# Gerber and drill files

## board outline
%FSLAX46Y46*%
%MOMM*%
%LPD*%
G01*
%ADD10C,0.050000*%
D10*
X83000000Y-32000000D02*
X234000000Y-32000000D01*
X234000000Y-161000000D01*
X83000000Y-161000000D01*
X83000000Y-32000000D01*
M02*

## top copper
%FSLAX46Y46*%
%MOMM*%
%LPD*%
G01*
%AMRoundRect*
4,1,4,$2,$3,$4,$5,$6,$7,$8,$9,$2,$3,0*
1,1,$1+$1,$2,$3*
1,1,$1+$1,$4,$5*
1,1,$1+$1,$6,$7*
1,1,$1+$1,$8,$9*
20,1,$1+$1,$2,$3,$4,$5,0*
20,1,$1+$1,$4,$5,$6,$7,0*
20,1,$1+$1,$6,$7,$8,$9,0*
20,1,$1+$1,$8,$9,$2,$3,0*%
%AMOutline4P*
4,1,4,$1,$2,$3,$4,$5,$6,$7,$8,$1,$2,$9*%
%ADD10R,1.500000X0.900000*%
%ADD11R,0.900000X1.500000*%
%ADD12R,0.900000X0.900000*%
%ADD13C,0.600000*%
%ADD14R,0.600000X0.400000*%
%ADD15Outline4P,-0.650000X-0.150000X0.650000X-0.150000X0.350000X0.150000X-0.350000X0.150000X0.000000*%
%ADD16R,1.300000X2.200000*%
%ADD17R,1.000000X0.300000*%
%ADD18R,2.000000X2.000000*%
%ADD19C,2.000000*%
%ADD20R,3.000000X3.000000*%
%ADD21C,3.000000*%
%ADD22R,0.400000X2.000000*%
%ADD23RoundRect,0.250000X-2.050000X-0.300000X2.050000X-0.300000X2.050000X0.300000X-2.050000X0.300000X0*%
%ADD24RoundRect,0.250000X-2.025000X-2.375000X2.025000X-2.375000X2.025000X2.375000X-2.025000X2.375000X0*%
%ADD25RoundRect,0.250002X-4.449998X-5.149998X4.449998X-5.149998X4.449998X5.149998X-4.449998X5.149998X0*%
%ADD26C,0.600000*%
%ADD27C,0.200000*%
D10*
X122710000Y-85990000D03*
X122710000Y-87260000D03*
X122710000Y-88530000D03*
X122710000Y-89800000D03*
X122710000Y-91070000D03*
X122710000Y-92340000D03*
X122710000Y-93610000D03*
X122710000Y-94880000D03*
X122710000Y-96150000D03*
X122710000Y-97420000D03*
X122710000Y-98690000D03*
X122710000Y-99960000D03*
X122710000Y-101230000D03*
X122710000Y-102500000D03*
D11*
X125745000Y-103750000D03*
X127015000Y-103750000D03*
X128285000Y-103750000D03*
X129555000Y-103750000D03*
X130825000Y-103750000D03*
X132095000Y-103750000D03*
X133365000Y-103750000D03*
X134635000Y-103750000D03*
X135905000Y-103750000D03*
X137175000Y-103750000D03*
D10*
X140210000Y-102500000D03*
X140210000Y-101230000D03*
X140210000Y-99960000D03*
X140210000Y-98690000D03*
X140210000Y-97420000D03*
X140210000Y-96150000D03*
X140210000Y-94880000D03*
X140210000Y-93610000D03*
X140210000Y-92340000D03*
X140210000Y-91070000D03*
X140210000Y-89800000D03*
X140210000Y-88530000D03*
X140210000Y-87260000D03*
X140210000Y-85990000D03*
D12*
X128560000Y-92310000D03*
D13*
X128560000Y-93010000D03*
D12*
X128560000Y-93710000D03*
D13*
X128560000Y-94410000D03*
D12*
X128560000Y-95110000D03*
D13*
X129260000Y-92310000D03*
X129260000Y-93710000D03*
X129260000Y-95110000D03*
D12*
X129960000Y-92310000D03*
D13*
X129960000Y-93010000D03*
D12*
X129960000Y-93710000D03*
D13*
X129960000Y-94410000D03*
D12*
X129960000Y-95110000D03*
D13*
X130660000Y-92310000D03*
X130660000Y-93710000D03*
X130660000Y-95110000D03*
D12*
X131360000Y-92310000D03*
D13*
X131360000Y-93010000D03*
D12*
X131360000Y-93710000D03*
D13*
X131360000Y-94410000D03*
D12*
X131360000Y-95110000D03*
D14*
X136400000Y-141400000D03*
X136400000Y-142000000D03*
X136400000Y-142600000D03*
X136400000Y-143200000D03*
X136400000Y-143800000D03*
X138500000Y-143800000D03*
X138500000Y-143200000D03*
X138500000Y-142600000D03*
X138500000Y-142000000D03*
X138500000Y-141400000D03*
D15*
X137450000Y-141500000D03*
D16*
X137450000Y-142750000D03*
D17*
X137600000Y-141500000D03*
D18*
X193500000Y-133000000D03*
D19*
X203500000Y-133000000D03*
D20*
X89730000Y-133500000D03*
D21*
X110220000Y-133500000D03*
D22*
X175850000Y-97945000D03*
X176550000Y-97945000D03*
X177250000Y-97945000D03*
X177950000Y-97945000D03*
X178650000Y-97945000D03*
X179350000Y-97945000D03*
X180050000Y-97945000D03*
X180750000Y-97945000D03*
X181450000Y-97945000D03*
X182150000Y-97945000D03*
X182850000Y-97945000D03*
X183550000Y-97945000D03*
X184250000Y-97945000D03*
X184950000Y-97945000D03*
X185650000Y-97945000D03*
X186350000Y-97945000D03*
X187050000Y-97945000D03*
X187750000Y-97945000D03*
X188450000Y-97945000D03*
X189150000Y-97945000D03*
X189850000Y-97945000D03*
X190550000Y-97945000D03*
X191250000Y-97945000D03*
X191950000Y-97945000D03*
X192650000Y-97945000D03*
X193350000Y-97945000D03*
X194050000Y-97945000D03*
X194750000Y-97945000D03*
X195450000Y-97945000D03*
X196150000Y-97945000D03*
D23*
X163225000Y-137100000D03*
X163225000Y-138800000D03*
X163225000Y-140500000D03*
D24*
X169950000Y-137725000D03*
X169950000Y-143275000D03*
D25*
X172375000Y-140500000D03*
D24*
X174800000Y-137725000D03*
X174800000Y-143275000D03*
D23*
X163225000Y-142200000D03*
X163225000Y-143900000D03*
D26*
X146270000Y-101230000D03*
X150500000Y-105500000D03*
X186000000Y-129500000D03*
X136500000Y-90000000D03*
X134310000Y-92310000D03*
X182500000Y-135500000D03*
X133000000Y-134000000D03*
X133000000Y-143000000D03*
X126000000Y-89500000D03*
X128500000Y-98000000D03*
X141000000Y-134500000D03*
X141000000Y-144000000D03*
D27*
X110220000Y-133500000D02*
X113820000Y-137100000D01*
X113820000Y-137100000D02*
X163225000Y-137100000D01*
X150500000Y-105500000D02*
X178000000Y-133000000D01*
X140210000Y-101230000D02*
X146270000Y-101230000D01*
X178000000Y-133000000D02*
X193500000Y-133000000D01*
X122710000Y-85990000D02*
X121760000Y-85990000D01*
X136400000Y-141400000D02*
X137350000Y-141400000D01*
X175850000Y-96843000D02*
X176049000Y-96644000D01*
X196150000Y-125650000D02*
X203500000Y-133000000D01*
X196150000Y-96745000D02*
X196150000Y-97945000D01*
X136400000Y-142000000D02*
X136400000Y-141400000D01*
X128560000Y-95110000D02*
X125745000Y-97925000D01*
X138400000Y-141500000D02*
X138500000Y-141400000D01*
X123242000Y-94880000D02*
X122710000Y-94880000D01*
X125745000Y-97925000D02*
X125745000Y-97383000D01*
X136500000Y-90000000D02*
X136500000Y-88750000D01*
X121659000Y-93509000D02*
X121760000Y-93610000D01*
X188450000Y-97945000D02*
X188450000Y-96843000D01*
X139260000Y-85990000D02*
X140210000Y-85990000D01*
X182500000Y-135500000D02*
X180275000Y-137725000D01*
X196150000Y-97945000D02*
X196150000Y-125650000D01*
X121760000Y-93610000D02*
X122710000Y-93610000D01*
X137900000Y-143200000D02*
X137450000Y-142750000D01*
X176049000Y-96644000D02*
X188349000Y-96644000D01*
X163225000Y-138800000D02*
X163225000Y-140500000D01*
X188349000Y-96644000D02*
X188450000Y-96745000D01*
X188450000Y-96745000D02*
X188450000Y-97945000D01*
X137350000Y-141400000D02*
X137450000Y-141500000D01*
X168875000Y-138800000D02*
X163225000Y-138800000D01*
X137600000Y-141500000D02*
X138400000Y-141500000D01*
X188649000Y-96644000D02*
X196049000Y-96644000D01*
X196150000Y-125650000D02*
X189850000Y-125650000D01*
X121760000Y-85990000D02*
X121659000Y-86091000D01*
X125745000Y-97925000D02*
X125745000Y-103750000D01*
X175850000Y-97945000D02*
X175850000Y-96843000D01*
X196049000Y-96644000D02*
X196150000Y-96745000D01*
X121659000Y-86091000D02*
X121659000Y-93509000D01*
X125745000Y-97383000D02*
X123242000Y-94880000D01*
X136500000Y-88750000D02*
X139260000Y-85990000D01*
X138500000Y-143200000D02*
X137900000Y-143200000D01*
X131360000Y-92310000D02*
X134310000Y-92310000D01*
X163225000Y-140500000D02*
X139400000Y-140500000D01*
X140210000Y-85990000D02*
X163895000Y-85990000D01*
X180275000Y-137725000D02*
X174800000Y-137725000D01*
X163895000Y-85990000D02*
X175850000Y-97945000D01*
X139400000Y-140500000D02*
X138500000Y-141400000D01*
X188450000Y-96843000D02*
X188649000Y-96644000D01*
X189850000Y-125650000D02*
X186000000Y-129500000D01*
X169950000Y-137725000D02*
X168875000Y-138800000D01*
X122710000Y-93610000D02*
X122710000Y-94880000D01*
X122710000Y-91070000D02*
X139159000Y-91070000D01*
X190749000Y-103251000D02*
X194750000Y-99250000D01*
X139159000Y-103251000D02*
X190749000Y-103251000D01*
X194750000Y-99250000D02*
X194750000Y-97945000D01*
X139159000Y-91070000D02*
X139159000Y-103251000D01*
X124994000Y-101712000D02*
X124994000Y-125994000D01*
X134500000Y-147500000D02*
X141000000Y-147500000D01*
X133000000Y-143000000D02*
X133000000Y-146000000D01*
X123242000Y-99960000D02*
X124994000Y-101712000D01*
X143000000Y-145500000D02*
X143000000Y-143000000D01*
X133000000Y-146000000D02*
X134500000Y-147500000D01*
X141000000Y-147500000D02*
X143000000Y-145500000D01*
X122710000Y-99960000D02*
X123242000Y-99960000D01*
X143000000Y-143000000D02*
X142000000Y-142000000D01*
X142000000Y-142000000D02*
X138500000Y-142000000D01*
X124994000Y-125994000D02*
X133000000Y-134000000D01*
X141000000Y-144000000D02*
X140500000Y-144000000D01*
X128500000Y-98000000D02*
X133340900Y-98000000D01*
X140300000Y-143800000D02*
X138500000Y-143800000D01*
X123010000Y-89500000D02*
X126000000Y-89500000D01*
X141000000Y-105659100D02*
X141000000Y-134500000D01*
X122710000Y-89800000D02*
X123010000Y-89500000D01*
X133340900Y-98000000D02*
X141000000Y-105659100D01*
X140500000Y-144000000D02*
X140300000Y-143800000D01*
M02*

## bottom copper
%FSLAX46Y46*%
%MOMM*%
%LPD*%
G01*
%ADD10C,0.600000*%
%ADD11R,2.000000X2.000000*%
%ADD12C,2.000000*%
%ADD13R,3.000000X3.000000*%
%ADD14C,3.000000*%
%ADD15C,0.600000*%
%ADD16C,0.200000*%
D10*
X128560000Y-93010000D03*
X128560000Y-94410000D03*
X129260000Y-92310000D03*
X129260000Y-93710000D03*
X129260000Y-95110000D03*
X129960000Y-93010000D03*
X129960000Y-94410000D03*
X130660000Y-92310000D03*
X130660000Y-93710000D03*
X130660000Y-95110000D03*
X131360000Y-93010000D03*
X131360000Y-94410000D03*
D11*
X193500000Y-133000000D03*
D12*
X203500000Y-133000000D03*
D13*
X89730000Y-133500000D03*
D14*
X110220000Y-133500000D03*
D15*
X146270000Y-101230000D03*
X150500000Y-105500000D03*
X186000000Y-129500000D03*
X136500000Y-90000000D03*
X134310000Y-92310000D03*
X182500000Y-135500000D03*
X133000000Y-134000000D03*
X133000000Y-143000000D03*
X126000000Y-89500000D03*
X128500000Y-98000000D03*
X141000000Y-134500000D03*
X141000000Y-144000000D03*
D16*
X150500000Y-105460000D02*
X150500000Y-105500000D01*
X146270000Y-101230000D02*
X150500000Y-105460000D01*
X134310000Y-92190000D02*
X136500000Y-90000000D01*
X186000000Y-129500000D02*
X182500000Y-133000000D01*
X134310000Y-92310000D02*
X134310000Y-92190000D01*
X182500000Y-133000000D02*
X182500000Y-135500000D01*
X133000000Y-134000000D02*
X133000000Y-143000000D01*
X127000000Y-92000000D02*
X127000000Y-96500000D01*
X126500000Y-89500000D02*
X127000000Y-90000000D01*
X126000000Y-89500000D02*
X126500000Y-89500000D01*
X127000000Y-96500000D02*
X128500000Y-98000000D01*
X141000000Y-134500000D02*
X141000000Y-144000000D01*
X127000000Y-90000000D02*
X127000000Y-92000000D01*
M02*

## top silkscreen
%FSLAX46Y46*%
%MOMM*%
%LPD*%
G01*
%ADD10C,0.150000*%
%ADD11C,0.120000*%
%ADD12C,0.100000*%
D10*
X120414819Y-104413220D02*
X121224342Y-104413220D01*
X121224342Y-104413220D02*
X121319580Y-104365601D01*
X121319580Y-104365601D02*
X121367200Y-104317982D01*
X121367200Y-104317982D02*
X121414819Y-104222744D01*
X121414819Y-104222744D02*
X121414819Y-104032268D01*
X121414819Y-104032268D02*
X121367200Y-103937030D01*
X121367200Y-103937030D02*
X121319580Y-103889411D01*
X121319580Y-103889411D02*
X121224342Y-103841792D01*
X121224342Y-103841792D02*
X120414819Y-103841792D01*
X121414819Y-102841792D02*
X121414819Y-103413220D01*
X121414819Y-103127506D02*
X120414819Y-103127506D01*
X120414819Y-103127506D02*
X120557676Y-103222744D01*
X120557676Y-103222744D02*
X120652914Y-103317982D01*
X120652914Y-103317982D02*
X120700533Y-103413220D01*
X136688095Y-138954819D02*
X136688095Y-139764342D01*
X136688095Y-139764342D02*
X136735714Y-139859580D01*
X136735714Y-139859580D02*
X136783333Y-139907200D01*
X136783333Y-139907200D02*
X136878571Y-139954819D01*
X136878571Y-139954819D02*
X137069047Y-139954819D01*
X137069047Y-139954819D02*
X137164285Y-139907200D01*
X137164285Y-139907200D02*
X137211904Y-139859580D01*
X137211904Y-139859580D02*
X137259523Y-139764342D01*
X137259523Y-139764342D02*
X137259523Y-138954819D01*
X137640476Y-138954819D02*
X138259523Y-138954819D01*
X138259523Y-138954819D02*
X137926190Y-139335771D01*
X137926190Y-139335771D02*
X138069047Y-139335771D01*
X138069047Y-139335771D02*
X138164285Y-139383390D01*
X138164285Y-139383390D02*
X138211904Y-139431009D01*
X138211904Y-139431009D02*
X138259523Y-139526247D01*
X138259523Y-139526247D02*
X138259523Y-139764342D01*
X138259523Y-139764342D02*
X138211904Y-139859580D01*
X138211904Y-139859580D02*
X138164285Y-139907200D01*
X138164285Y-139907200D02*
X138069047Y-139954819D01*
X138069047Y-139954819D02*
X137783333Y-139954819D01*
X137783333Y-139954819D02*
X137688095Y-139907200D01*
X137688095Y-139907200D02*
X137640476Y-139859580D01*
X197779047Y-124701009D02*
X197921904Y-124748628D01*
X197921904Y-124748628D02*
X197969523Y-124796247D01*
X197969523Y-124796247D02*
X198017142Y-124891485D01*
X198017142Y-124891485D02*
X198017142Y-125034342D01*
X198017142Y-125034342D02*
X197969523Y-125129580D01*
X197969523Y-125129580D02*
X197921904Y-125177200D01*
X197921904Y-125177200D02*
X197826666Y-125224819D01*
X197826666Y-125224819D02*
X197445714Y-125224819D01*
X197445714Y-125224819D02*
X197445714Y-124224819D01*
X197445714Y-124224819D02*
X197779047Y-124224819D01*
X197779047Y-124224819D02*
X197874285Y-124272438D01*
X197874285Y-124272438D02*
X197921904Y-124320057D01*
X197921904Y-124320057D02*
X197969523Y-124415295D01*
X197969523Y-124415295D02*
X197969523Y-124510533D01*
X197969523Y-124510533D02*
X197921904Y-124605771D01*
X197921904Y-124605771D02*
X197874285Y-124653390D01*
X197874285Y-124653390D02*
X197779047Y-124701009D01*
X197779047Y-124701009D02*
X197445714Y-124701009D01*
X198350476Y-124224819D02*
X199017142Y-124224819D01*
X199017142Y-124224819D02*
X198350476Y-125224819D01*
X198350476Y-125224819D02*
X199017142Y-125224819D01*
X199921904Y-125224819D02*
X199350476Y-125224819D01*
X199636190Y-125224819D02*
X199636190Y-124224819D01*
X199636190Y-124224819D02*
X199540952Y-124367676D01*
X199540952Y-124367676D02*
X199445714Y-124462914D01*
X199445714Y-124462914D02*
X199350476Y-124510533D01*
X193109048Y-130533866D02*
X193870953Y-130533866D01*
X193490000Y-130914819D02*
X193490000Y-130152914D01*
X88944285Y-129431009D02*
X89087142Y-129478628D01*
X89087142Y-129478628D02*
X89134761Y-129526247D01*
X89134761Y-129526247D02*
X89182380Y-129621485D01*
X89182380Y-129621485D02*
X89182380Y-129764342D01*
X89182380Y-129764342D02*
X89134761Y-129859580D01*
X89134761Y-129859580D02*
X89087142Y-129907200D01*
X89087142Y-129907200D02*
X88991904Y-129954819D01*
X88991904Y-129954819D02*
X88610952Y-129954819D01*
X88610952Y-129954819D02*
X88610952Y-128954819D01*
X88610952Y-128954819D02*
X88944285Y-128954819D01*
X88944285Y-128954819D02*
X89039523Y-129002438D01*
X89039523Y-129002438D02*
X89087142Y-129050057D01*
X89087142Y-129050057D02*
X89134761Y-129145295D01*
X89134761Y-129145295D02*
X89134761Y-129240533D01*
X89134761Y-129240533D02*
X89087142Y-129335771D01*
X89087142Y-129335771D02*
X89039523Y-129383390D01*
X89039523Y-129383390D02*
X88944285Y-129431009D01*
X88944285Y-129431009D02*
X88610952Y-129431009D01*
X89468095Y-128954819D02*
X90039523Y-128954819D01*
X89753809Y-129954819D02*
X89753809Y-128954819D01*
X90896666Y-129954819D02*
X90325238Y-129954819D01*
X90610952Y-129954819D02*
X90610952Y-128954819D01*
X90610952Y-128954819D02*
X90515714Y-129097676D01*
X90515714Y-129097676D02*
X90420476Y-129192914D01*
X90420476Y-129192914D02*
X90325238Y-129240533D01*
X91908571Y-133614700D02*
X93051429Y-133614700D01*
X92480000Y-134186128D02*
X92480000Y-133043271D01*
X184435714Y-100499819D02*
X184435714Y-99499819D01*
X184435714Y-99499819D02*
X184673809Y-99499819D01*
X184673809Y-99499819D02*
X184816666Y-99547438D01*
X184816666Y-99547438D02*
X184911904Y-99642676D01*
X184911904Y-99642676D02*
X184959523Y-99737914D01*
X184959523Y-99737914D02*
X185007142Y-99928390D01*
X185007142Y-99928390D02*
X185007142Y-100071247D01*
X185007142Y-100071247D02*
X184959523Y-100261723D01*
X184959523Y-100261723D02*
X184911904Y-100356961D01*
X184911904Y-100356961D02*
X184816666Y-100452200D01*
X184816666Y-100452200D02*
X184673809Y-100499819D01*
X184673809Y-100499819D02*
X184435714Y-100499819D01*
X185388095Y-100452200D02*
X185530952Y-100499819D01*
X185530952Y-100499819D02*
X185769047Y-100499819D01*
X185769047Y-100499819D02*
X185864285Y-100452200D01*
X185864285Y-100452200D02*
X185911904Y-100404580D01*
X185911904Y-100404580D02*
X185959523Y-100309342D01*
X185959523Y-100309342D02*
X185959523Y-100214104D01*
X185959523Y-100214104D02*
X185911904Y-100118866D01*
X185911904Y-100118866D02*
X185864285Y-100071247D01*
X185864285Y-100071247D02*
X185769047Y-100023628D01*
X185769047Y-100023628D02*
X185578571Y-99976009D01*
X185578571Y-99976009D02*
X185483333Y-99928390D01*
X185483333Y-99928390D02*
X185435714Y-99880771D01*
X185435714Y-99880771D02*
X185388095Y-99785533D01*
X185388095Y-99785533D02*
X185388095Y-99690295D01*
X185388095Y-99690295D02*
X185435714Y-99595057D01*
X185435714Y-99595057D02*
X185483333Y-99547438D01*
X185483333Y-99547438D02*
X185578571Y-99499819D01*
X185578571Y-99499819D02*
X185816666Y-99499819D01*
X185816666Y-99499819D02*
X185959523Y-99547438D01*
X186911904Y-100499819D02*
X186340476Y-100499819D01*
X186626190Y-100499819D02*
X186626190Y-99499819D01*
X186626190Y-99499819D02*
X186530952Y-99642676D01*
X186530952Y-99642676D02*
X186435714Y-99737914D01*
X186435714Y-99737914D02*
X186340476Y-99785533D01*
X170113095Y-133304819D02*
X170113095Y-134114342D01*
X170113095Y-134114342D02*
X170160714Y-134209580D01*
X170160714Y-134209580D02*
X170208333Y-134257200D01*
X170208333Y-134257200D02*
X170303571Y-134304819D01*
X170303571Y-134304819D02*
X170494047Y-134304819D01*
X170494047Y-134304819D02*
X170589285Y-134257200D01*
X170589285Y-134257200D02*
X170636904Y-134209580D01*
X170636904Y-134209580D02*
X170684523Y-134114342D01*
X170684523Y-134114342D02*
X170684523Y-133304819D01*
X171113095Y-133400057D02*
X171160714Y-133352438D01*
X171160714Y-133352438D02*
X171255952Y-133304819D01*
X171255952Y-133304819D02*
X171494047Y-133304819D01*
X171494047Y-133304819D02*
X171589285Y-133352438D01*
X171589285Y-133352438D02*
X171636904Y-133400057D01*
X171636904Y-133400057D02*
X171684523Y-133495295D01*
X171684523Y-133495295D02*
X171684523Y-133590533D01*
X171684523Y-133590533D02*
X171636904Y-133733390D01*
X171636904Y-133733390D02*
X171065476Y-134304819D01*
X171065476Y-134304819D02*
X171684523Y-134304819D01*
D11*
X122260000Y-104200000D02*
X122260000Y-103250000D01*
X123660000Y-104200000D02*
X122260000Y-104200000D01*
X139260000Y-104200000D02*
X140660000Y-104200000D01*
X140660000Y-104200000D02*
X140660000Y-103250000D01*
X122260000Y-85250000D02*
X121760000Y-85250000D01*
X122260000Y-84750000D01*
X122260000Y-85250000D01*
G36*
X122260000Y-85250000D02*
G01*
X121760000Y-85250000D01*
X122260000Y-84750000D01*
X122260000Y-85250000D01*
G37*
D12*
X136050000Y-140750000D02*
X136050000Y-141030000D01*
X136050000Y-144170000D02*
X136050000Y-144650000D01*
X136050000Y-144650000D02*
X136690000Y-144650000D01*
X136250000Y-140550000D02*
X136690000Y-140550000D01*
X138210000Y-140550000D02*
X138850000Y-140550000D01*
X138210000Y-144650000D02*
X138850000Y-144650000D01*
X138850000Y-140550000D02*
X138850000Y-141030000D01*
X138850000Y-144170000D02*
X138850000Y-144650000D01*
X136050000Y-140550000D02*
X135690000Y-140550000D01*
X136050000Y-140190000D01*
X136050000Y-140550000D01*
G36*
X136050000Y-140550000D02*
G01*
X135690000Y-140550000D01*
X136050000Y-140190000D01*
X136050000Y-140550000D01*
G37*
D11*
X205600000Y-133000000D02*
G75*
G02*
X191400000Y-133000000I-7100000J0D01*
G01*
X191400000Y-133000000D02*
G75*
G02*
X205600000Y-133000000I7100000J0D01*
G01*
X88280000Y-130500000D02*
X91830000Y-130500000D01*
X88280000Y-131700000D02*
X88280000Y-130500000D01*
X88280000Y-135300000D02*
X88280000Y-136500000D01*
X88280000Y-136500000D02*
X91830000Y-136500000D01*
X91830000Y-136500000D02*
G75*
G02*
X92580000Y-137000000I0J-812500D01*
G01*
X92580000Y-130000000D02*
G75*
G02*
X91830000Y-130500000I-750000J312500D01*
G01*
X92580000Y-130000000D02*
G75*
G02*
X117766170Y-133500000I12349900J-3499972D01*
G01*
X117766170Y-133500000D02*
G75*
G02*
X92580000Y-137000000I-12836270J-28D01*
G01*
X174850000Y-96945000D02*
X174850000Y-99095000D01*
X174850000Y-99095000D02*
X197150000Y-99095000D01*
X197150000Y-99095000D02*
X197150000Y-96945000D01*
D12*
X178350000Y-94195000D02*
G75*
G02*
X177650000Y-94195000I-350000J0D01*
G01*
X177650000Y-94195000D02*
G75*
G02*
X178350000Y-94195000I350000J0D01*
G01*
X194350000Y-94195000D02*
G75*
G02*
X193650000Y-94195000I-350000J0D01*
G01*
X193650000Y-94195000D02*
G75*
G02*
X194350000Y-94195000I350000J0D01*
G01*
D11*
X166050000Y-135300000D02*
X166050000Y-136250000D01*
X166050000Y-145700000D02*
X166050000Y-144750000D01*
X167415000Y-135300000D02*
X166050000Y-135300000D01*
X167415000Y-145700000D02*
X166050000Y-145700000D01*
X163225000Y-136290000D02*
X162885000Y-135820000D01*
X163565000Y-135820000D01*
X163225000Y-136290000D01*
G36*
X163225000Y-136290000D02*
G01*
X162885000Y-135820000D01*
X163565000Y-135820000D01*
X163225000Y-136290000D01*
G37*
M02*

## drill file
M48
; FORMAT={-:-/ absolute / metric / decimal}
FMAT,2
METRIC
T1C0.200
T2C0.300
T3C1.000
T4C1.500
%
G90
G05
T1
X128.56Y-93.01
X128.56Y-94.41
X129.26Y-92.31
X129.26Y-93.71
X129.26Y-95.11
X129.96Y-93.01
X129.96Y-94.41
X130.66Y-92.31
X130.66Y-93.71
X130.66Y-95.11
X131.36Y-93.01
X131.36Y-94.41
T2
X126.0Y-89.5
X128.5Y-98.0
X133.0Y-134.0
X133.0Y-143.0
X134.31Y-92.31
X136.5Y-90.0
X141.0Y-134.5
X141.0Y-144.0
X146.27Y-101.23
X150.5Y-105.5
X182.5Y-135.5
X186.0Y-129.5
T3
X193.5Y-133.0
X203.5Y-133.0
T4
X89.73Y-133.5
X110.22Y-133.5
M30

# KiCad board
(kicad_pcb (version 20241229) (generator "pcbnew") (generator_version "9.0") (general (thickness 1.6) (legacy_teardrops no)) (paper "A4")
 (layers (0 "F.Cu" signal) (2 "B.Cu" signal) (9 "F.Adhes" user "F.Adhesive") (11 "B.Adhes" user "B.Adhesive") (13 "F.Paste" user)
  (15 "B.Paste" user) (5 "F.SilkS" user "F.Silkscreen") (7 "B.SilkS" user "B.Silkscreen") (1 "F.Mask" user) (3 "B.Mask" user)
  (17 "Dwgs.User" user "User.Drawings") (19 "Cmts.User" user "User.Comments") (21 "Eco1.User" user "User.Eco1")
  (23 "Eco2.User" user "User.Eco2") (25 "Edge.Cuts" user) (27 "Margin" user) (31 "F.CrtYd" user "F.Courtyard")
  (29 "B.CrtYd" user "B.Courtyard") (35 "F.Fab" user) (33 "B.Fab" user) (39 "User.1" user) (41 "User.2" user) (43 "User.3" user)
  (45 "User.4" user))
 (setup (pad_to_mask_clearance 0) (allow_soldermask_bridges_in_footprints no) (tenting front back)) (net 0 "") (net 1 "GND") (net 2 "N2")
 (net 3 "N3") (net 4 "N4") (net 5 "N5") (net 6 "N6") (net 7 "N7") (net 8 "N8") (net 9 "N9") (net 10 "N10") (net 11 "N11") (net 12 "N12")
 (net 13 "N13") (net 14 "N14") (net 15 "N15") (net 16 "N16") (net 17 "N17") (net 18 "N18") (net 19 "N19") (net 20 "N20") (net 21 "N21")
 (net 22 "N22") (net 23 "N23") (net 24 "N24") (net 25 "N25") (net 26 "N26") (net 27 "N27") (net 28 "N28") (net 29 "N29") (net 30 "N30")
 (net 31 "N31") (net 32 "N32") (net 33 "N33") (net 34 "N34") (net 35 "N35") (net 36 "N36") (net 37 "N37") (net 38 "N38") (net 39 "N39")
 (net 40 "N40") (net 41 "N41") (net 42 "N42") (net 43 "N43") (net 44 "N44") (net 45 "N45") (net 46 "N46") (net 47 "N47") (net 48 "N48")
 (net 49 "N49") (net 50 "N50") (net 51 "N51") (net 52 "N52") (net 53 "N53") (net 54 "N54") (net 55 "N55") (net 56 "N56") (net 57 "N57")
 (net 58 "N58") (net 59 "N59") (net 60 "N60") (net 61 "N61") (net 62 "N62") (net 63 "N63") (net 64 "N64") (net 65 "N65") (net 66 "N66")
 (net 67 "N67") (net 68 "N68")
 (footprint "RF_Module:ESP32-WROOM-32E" (layer "F.Cu") (at 131.46 91.25)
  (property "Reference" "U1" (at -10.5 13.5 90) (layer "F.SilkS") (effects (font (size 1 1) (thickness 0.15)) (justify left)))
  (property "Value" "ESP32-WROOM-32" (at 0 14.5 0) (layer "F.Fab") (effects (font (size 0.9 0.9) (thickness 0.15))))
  (fp_line (start -9.2 12.95) (end -9.2 12) (stroke (width 0.12) (type solid)) (layer "F.SilkS"))
  (fp_line (start -7.8 12.95) (end -9.2 12.95) (stroke (width 0.12) (type solid)) (layer "F.SilkS"))
  (fp_line (start 7.8 12.95) (end 9.2 12.95) (stroke (width 0.12) (type solid)) (layer "F.SilkS"))
  (fp_line (start 9.2 12.95) (end 9.2 12) (stroke (width 0.12) (type solid)) (layer "F.SilkS"))
  (fp_poly (pts (xy -9.2 -6) (xy -9.7 -6) (xy -9.2 -6.5) (xy -9.2 -6)) (stroke (width 0.12) (type solid)) (fill yes) (layer "F.SilkS"))
  (pad "1" smd rect (at -8.75 -5.26) (size 1.5 0.9) (layers "F.Cu" "F.Mask" "F.Paste") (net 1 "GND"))
  (pad "2" smd rect (at -8.75 -3.99) (size 1.5 0.9) (layers "F.Cu" "F.Mask" "F.Paste") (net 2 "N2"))
  (pad "3" smd rect (at -8.75 -2.72) (size 1.5 0.9) (layers "F.Cu" "F.Mask" "F.Paste") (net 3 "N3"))
  (pad "4" smd rect (at -8.75 -1.45) (size 1.5 0.9) (layers "F.Cu" "F.Mask" "F.Paste") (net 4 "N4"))
  (pad "5" smd rect (at -8.75 -0.18) (size 1.5 0.9) (layers "F.Cu" "F.Mask" "F.Paste") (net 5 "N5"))
  (pad "6" smd rect (at -8.75 1.09) (size 1.5 0.9) (layers "F.Cu" "F.Mask" "F.Paste") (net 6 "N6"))
  (pad "7" smd rect (at -8.75 2.36) (size 1.5 0.9) (layers "F.Cu" "F.Mask" "F.Paste") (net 1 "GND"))
  (pad "8" smd rect (at -8.75 3.63) (size 1.5 0.9) (layers "F.Cu" "F.Mask" "F.Paste") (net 1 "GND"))
  (pad "9" smd rect (at -8.75 4.9) (size 1.5 0.9) (layers "F.Cu" "F.Mask" "F.Paste") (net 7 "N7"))
  (pad "10" smd rect (at -8.75 6.17) (size 1.5 0.9) (layers "F.Cu" "F.Mask" "F.Paste") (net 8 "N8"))
  (pad "11" smd rect (at -8.75 7.44) (size 1.5 0.9) (layers "F.Cu" "F.Mask" "F.Paste") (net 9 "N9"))
  (pad "12" smd rect (at -8.75 8.71) (size 1.5 0.9) (layers "F.Cu" "F.Mask" "F.Paste") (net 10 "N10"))
  (pad "13" smd rect (at -8.75 9.98) (size 1.5 0.9) (layers "F.Cu" "F.Mask" "F.Paste") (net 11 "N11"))
  (pad "14" smd rect (at -8.75 11.25) (size 1.5 0.9) (layers "F.Cu" "F.Mask" "F.Paste") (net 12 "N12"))
  (pad "15" smd rect (at -5.715 12.5 90) (size 1.5 0.9) (layers "F.Cu" "F.Mask" "F.Paste") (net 1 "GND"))
  (pad "16" smd rect (at -4.445 12.5 90) (size 1.5 0.9) (layers "F.Cu" "F.Mask" "F.Paste") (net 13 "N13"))
  (pad "17" smd rect (at -3.175 12.5 90) (size 1.5 0.9) (layers "F.Cu" "F.Mask" "F.Paste") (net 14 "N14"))
  (pad "18" smd rect (at -1.905 12.5 90) (size 1.5 0.9) (layers "F.Cu" "F.Mask" "F.Paste") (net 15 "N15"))
  (pad "19" smd rect (at -0.635 12.5 90) (size 1.5 0.9) (layers "F.Cu" "F.Mask" "F.Paste") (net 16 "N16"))
  (pad "20" smd rect (at 0.635 12.5 90) (size 1.5 0.9) (layers "F.Cu" "F.Mask" "F.Paste") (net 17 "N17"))
  (pad "21" smd rect (at 1.905 12.5 90) (size 1.5 0.9) (layers "F.Cu" "F.Mask" "F.Paste") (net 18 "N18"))
  (pad "22" smd rect (at 3.175 12.5 90) (size 1.5 0.9) (layers "F.Cu" "F.Mask" "F.Paste") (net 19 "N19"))
  (pad "23" smd rect (at 4.445 12.5 90) (size 1.5 0.9) (layers "F.Cu" "F.Mask" "F.Paste") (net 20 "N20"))
  (pad "24" smd rect (at 5.715 12.5 90) (size 1.5 0.9) (layers "F.Cu" "F.Mask" "F.Paste") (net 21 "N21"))
  (pad "25" smd rect (at 8.75 11.25) (size 1.5 0.9) (layers "F.Cu" "F.Mask" "F.Paste") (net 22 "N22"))
  (pad "26" smd rect (at 8.75 9.98) (size 1.5 0.9) (layers "F.Cu" "F.Mask" "F.Paste") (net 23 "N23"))
  (pad "27" smd rect (at 8.75 8.71) (size 1.5 0.9) (layers "F.Cu" "F.Mask" "F.Paste") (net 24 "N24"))
  (pad "28" smd rect (at 8.75 7.44) (size 1.5 0.9) (layers "F.Cu" "F.Mask" "F.Paste") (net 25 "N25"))
  (pad "29" smd rect (at 8.75 6.17) (size 1.5 0.9) (layers "F.Cu" "F.Mask" "F.Paste") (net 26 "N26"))
  (pad "30" smd rect (at 8.75 4.9) (size 1.5 0.9) (layers "F.Cu" "F.Mask" "F.Paste") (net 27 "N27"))
  (pad "31" smd rect (at 8.75 3.63) (size 1.5 0.9) (layers "F.Cu" "F.Mask" "F.Paste") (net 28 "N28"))
  (pad "32" smd rect (at 8.75 2.36) (size 1.5 0.9) (layers "F.Cu" "F.Mask" "F.Paste") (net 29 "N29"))
  (pad "33" smd rect (at 8.75 1.09) (size 1.5 0.9) (layers "F.Cu" "F.Mask" "F.Paste") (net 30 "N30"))
  (pad "34" smd rect (at 8.75 -0.18) (size 1.5 0.9) (layers "F.Cu" "F.Mask" "F.Paste") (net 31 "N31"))
  (pad "35" smd rect (at 8.75 -1.45) (size 1.5 0.9) (layers "F.Cu" "F.Mask" "F.Paste") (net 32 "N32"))
  (pad "36" smd rect (at 8.75 -2.72) (size 1.5 0.9) (layers "F.Cu" "F.Mask" "F.Paste") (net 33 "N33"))
  (pad "37" smd rect (at 8.75 -3.99) (size 1.5 0.9) (layers "F.Cu" "F.Mask" "F.Paste") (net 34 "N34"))
  (pad "38" smd rect (at 8.75 -5.26) (size 1.5 0.9) (layers "F.Cu" "F.Mask" "F.Paste") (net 1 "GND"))
  (pad "39" smd rect (at -2.9 1.06) (size 0.9 0.9) (layers "F.Cu" "F.Mask" "F.Paste") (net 1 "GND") (zone_connect 2))
  (pad "39" thru_hole circle (at -2.9 1.76) (size 0.6 0.6) (drill 0.2) (layers "*.Cu" "*.Mask") (remove_unused_layers no) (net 1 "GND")
   (zone_connect 2))
  (pad "39" smd rect (at -2.9 2.46) (size 0.9 0.9) (layers "F.Cu" "F.Mask" "F.Paste") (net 1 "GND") (zone_connect 2))
  (pad "39" thru_hole circle (at -2.9 3.16) (size 0.6 0.6) (drill 0.2) (layers "*.Cu" "*.Mask") (remove_unused_layers no) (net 1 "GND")
   (zone_connect 2))
  (pad "39" smd rect (at -2.9 3.86) (size 0.9 0.9) (layers "F.Cu" "F.Mask" "F.Paste") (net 1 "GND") (zone_connect 2))
  (pad "39" thru_hole circle (at -2.2 1.06) (size 0.6 0.6) (drill 0.2) (layers "*.Cu" "*.Mask") (remove_unused_layers no) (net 1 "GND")
   (zone_connect 2))
  (pad "39" thru_hole circle (at -2.2 2.46) (size 0.6 0.6) (drill 0.2) (layers "*.Cu" "*.Mask") (remove_unused_layers no) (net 1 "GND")
   (zone_connect 2))
  (pad "39" thru_hole circle (at -2.2 3.86) (size 0.6 0.6) (drill 0.2) (layers "*.Cu" "*.Mask") (remove_unused_layers no) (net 1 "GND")
   (zone_connect 2))
  (pad "39" smd rect (at -1.5 1.06) (size 0.9 0.9) (layers "F.Cu" "F.Mask" "F.Paste") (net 1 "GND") (zone_connect 2))
  (pad "39" thru_hole circle (at -1.5 1.76) (size 0.6 0.6) (drill 0.2) (layers "*.Cu" "*.Mask") (remove_unused_layers no) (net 1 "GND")
   (zone_connect 2))
  (pad "39" smd rect (at -1.5 2.46) (size 0.9 0.9) (layers "F.Cu" "F.Mask" "F.Paste") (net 1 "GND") (zone_connect 2))
  (pad "39" thru_hole circle (at -1.5 3.16) (size 0.6 0.6) (drill 0.2) (layers "*.Cu" "*.Mask") (remove_unused_layers no) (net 1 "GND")
   (zone_connect 2))
  (pad "39" smd rect (at -1.5 3.86) (size 0.9 0.9) (layers "F.Cu" "F.Mask" "F.Paste") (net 1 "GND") (zone_connect 2))
  (pad "39" thru_hole circle (at -0.8 1.06) (size 0.6 0.6) (drill 0.2) (layers "*.Cu" "*.Mask") (remove_unused_layers no) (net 1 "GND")
   (zone_connect 2))
  (pad "39" thru_hole circle (at -0.8 2.46) (size 0.6 0.6) (drill 0.2) (layers "*.Cu" "*.Mask") (remove_unused_layers no) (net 1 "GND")
   (zone_connect 2))
  (pad "39" thru_hole circle (at -0.8 3.86) (size 0.6 0.6) (drill 0.2) (layers "*.Cu" "*.Mask") (remove_unused_layers no) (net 1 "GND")
   (zone_connect 2))
  (pad "39" smd rect (at -0.1 1.06) (size 0.9 0.9) (layers "F.Cu" "F.Mask" "F.Paste") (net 1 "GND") (zone_connect 2))
  (pad "39" thru_hole circle (at -0.1 1.76) (size 0.6 0.6) (drill 0.2) (layers "*.Cu" "*.Mask") (remove_unused_layers no) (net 1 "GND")
   (zone_connect 2))
  (pad "39" smd rect (at -0.1 2.46) (size 0.9 0.9) (layers "F.Cu" "F.Mask" "F.Paste") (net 1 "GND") (zone_connect 2))
  (pad "39" thru_hole circle (at -0.1 3.16) (size 0.6 0.6) (drill 0.2) (layers "*.Cu" "*.Mask") (remove_unused_layers no) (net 1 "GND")
   (zone_connect 2))
  (pad "39" smd rect (at -0.1 3.86) (size 0.9 0.9) (layers "F.Cu" "F.Mask" "F.Paste") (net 1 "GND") (zone_connect 2))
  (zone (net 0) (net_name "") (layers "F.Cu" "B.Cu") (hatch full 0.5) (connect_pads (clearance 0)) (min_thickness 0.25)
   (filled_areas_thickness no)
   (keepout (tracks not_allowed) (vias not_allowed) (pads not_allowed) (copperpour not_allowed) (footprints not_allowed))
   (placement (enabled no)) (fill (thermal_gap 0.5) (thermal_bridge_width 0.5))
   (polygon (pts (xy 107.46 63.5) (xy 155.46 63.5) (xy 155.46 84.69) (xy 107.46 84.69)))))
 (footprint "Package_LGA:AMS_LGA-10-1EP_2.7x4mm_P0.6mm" (layer "F.Cu") (at 137.45 142.6)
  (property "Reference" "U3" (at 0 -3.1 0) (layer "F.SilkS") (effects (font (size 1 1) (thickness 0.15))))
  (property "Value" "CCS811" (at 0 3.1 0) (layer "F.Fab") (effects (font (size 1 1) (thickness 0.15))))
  (fp_line (start -1.4 -1.85) (end -1.4 -1.57) (stroke (width 0.1) (type solid)) (layer "F.SilkS"))
  (fp_line (start -1.4 1.57) (end -1.4 2.05) (stroke (width 0.1) (type solid)) (layer "F.SilkS"))
  (fp_line (start -1.4 2.05) (end -0.76 2.05) (stroke (width 0.1) (type solid)) (layer "F.SilkS"))
  (fp_line (start -1.2 -2.05) (end -0.76 -2.05) (stroke (width 0.1) (type solid)) (layer "F.SilkS"))
  (fp_line (start 0.76 -2.05) (end 1.4 -2.05) (stroke (width 0.1) (type solid)) (layer "F.SilkS"))
  (fp_line (start 0.76 2.05) (end 1.4 2.05) (stroke (width 0.1) (type solid)) (layer "F.SilkS"))
  (fp_line (start 1.4 -2.05) (end 1.4 -1.57) (stroke (width 0.1) (type solid)) (layer "F.SilkS"))
  (fp_line (start 1.4 1.57) (end 1.4 2.05) (stroke (width 0.1) (type solid)) (layer "F.SilkS"))
  (fp_poly
   (pts (xy -1.4 -2.05) (xy -1.76 -2.05) (xy -1.4 -2.41) (xy -1.4 -2.05)) (stroke (width 0.1) (type solid)) (fill yes) (layer "F.SilkS"))
  (pad "1" smd rect (at -1.05 -1.2) (size 0.6 0.4) (layers "F.Cu" "F.Mask" "F.Paste") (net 1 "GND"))
  (pad "2" smd rect (at -1.05 -0.6) (size 0.6 0.4) (layers "F.Cu" "F.Mask" "F.Paste") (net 1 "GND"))
  (pad "3" smd rect (at -1.05 0) (size 0.6 0.4) (layers "F.Cu" "F.Mask" "F.Paste") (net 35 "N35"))
  (pad "4" smd rect (at -1.05 0.6) (size 0.6 0.4) (layers "F.Cu" "F.Mask" "F.Paste") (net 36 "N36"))
  (pad "5" smd rect (at -1.05 1.2) (size 0.6 0.4) (layers "F.Cu" "F.Mask" "F.Paste") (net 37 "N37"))
  (pad "6" smd rect (at 1.05 1.2) (size 0.6 0.4) (layers "F.Cu" "F.Mask" "F.Paste") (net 4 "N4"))
  (pad "7" smd rect (at 1.05 0.6) (size 0.6 0.4) (layers "F.Cu" "F.Mask" "F.Paste") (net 1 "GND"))
  (pad "8" smd rect (at 1.05 0) (size 0.6 0.4) (layers "F.Cu" "F.Mask" "F.Paste") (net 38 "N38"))
  (pad "9" smd rect (at 1.05 -0.6) (size 0.6 0.4) (layers "F.Cu" "F.Mask" "F.Paste") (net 10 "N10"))
  (pad "10" smd rect (at 1.05 -1.2) (size 0.6 0.4) (layers "F.Cu" "F.Mask" "F.Paste") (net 1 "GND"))
  (pad "11" smd trapezoid (at 0 -1.1) (size 1 0.3) (rect_delta 0 0.3) (layers "F.Cu" "F.Mask" "F.Paste") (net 1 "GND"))
  (pad "11" smd rect (at 0 0.15) (size 1.3 2.2) (layers "F.Cu" "F.Mask" "F.Paste") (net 1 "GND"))
  (pad "11" smd rect (at 0.15 -1.1) (size 1 0.3) (layers "F.Cu" "F.Mask" "F.Paste") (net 1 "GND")))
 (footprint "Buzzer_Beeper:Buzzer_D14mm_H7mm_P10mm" (layer "F.Cu") (at 193.5 133)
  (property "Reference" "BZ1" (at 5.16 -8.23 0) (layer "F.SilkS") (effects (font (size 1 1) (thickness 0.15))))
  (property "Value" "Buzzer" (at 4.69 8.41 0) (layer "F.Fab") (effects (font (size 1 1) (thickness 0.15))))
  (fp_circle (center 5 0) (end 12.1 0) (stroke (width 0.12) (type solid)) (fill no) (layer "F.SilkS"))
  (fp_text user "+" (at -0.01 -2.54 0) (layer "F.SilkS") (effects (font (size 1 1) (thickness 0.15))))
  (pad "1" thru_hole rect (at 0 0) (size 2 2) (drill 1) (layers "*.Cu" "*.Mask") (remove_unused_layers no) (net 23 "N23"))
  (pad "2" thru_hole circle (at 10 0) (size 2 2) (drill 1) (layers "*.Cu" "*.Mask") (remove_unused_layers no) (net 1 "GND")))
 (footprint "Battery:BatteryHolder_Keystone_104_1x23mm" (layer "F.Cu") (at 89.73 133.5)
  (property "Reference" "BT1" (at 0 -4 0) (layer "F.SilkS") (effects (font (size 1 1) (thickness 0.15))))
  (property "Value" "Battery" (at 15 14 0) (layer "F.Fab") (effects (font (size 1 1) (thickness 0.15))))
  (fp_line (start -1.45 -3) (end 2.1 -3) (stroke (width 0.12) (type solid)) (layer "F.SilkS"))
  (fp_line (start -1.45 -1.8) (end -1.45 -3) (stroke (width 0.12) (type solid)) (layer "F.SilkS"))
  (fp_line (start -1.45 1.8) (end -1.45 3) (stroke (width 0.12) (type solid)) (layer "F.SilkS"))
  (fp_line (start -1.45 3) (end 2.1 3) (stroke (width 0.12) (type solid)) (layer "F.SilkS"))
  (fp_arc (start 2.1 3) (mid 2.550694 3.136459) (end 2.85 3.5) (stroke (width 0.12) (type solid)) (layer "F.SilkS"))
  (fp_arc (start 2.85 -3.5) (mid 2.550694 -3.136459) (end 2.1 -3) (stroke (width 0.12) (type solid)) (layer "F.SilkS"))
  (fp_arc (start 2.85 -3.5) (mid 16.966716 -12.714122) (end 28.03617 0) (stroke (width 0.12) (type solid)) (layer "F.SilkS"))
  (fp_arc (start 28.03617 0) (mid 16.966716 12.714122) (end 2.85 3.5) (stroke (width 0.12) (type solid)) (layer "F.SilkS"))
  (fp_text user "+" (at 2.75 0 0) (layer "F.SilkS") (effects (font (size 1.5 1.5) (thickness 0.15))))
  (pad "1" thru_hole rect (at 0 0) (size 3 3) (drill 1.5) (layers "*.Cu" "*.Mask") (remove_unused_layers no) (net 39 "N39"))
  (pad "2" thru_hole circle (at 20.49 0) (size 3 3) (drill 1.5) (layers "*.Cu" "*.Mask") (remove_unused_layers no) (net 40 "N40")))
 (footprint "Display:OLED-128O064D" (layer "F.Cu") (at 186 97.945)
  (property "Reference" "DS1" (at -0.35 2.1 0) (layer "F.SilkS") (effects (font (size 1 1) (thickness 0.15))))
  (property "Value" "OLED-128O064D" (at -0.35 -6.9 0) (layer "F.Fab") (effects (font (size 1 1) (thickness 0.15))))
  (fp_line (start -11.15 -1) (end -11.15 1.15) (stroke (width 0.12) (type solid)) (layer "F.SilkS"))
  (fp_line (start -11.15 1.15) (end 11.15 1.15) (stroke (width 0.12) (type solid)) (layer "F.SilkS"))
  (fp_line (start 11.15 1.15) (end 11.15 -1) (stroke (width 0.12) (type solid)) (layer "F.SilkS"))
  (fp_circle (center -8 -3.75) (end -7.65 -3.75) (stroke (width 0.1) (type solid)) (fill no) (layer "F.SilkS"))
  (fp_circle (center 8 -3.75) (end 8.35 -3.75) (stroke (width 0.1) (type solid)) (fill no) (layer "F.SilkS"))
  (pad "1" smd rect (at -10.15 0) (size 0.4 2) (layers "F.Cu" "F.Mask" "F.Paste") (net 1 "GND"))
  (pad "2" smd rect (at -9.45 0) (size 0.4 2) (layers "F.Cu" "F.Mask" "F.Paste") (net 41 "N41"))
  (pad "3" smd rect (at -8.75 0) (size 0.4 2) (layers "F.Cu" "F.Mask" "F.Paste") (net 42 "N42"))
  (pad "4" smd rect (at -8.05 0) (size 0.4 2) (layers "F.Cu" "F.Mask" "F.Paste") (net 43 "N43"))
  (pad "5" smd rect (at -7.35 0) (size 0.4 2) (layers "F.Cu" "F.Mask" "F.Paste") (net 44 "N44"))
  (pad "6" smd rect (at -6.65 0) (size 0.4 2) (layers "F.Cu" "F.Mask" "F.Paste") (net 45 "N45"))
  (pad "7" smd rect (at -5.95 0) (size 0.4 2) (layers "F.Cu" "F.Mask" "F.Paste") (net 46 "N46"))
  (pad "8" smd rect (at -5.25 0) (size 0.4 2) (layers "F.Cu" "F.Mask" "F.Paste") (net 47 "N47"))
  (pad "9" smd rect (at -4.55 0) (size 0.4 2) (layers "F.Cu" "F.Mask" "F.Paste") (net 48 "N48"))
  (pad "10" smd rect (at -3.85 0) (size 0.4 2) (layers "F.Cu" "F.Mask" "F.Paste") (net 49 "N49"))
  (pad "11" smd rect (at -3.15 0) (size 0.4 2) (layers "F.Cu" "F.Mask" "F.Paste") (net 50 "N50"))
  (pad "12" smd rect (at -2.45 0) (size 0.4 2) (layers "F.Cu" "F.Mask" "F.Paste") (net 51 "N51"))
  (pad "13" smd rect (at -1.75 0) (size 0.4 2) (layers "F.Cu" "F.Mask" "F.Paste") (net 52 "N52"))
  (pad "14" smd rect (at -1.05 0) (size 0.4 2) (layers "F.Cu" "F.Mask" "F.Paste") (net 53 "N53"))
  (pad "15" smd rect (at -0.35 0) (size 0.4 2) (layers "F.Cu" "F.Mask" "F.Paste") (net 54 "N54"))
  (pad "16" smd rect (at 0.35 0) (size 0.4 2) (layers "F.Cu" "F.Mask" "F.Paste") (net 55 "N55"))
  (pad "17" smd rect (at 1.05 0) (size 0.4 2) (layers "F.Cu" "F.Mask" "F.Paste") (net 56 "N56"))
  (pad "18" smd rect (at 1.75 0) (size 0.4 2) (layers "F.Cu" "F.Mask" "F.Paste") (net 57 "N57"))
  (pad "19" smd rect (at 2.45 0) (size 0.4 2) (layers "F.Cu" "F.Mask" "F.Paste") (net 1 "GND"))
  (pad "20" smd rect (at 3.15 0) (size 0.4 2) (layers "F.Cu" "F.Mask" "F.Paste") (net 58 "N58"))
  (pad "21" smd rect (at 3.85 0) (size 0.4 2) (layers "F.Cu" "F.Mask" "F.Paste") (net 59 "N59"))
  (pad "22" smd rect (at 4.55 0) (size 0.4 2) (layers "F.Cu" "F.Mask" "F.Paste") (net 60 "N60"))
  (pad "23" smd rect (at 5.25 0) (size 0.4 2) (layers "F.Cu" "F.Mask" "F.Paste") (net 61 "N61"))
  (pad "24" smd rect (at 5.95 0) (size 0.4 2) (layers "F.Cu" "F.Mask" "F.Paste") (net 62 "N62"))
  (pad "25" smd rect (at 6.65 0) (size 0.4 2) (layers "F.Cu" "F.Mask" "F.Paste") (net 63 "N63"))
  (pad "26" smd rect (at 7.35 0) (size 0.4 2) (layers "F.Cu" "F.Mask" "F.Paste") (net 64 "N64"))
  (pad "27" smd rect (at 8.05 0) (size 0.4 2) (layers "F.Cu" "F.Mask" "F.Paste") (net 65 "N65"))
  (pad "28" smd rect (at 8.75 0) (size 0.4 2) (layers "F.Cu" "F.Mask" "F.Paste") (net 5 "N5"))
  (pad "29" smd rect (at 9.45 0) (size 0.4 2) (layers "F.Cu" "F.Mask" "F.Paste") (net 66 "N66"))
  (pad "30" smd rect (at 10.15 0) (size 0.4 2) (layers "F.Cu" "F.Mask" "F.Paste") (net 1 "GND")))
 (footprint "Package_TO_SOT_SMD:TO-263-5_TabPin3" (layer "F.Cu") (at 170.875 140.5)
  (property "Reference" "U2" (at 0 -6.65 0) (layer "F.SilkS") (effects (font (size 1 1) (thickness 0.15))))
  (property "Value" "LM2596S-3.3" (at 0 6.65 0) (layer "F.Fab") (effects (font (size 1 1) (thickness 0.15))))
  (fp_line (start -4.825 -5.2) (end -4.825 -4.25) (stroke (width 0.12) (type solid)) (layer "F.SilkS"))
  (fp_line (start -4.825 5.2) (end -4.825 4.25) (stroke (width 0.12) (type solid)) (layer "F.SilkS"))
  (fp_line (start -3.46 -5.2) (end -4.825 -5.2) (stroke (width 0.12) (type solid)) (layer "F.SilkS"))
  (fp_line (start -3.46 5.2) (end -4.825 5.2) (stroke (width 0.12) (type solid)) (layer "F.SilkS"))
  (fp_poly
   (pts (xy -7.65 -4.21) (xy -7.99 -4.68) (xy -7.31 -4.68) (xy -7.65 -4.21)) (stroke (width 0.12) (type solid)) (fill yes) (layer "F.SilkS"))
  (pad "1" smd roundrect (at -7.65 -3.4) (size 4.6 1.1) (layers "F.Cu" "F.Mask" "F.Paste") (roundrect_rratio 0.227273) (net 40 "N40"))
  (pad "2" smd roundrect (at -7.65 -1.7) (size 4.6 1.1) (layers "F.Cu" "F.Mask" "F.Paste") (roundrect_rratio 0.227273) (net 1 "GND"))
  (pad "3" smd roundrect (at -7.65 0) (size 4.6 1.1) (layers "F.Cu" "F.Mask" "F.Paste") (roundrect_rratio 0.227273) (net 1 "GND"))
  (pad "3" smd roundrect (at -0.925 -2.775) (size 4.55 5.25) (layers "F.Cu" "F.Paste") (roundrect_rratio 0.054945) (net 1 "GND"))
  (pad "3" smd roundrect (at -0.925 2.775) (size 4.55 5.25) (layers "F.Cu" "F.Paste") (roundrect_rratio 0.054945) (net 1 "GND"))
  (pad "3" smd roundrect (at 1.5 0) (size 9.4 10.8) (layers "F.Cu" "F.Mask") (roundrect_rratio 0.026596) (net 1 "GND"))
  (pad "3" smd roundrect (at 3.925 -2.775) (size 4.55 5.25) (layers "F.Cu" "F.Paste") (roundrect_rratio 0.054945) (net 1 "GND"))
  (pad "3" smd roundrect (at 3.925 2.775) (size 4.55 5.25) (layers "F.Cu" "F.Paste") (roundrect_rratio 0.054945) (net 1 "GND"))
  (pad "4" smd roundrect (at -7.65 1.7) (size 4.6 1.1) (layers "F.Cu" "F.Mask" "F.Paste") (roundrect_rratio 0.227273) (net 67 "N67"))
  (pad "5" smd roundrect (at -7.65 3.4) (size 4.6 1.1) (layers "F.Cu" "F.Mask" "F.Paste") (roundrect_rratio 0.227273) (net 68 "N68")))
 (gr_rect (start 83 32) (end 234 161) (stroke (width 0.05) (type default)) (fill no) (layer "Edge.Cuts"))
 (segment (start 110.22 133.5) (end 113.82 137.1) (width 0.2) (layer "F.Cu") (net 40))
 (segment (start 113.82 137.1) (end 163.225 137.1) (width 0.2) (layer "F.Cu") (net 40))
 (segment (start 150.5 105.5) (end 178 133) (width 0.2) (layer "F.Cu") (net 23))
 (segment (start 140.21 101.23) (end 146.27 101.23) (width 0.2) (layer "F.Cu") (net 23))
 (segment (start 178 133) (end 193.5 133) (width 0.2) (layer "F.Cu") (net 23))
 (via (at 146.27 101.23) (size 0.6) (drill 0.3) (layers "F.Cu" "B.Cu") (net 23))
 (via (at 150.5 105.5) (size 0.6) (drill 0.3) (layers "F.Cu" "B.Cu") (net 23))
 (segment (start 150.5 105.46) (end 150.5 105.5) (width 0.2) (layer "B.Cu") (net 23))
 (segment (start 146.27 101.23) (end 150.5 105.46) (width 0.2) (layer "B.Cu") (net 23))
 (segment (start 122.71 85.99) (end 121.76 85.99) (width 0.2) (layer "F.Cu") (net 1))
 (segment (start 136.4 141.4) (end 137.35 141.4) (width 0.2) (layer "F.Cu") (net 1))
 (segment (start 175.85 96.843) (end 176.049 96.644) (width 0.2) (layer "F.Cu") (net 1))
 (segment (start 196.15 125.65) (end 203.5 133) (width 0.2) (layer "F.Cu") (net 1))
 (segment (start 196.15 96.745) (end 196.15 97.945) (width 0.2) (layer "F.Cu") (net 1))
 (segment (start 136.4 142) (end 136.4 141.4) (width 0.2) (layer "F.Cu") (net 1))
 (segment (start 128.56 95.11) (end 125.745 97.925) (width 0.2) (layer "F.Cu") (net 1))
 (segment (start 138.4 141.5) (end 138.5 141.4) (width 0.2) (layer "F.Cu") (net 1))
 (segment (start 123.242 94.88) (end 122.71 94.88) (width 0.2) (layer "F.Cu") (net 1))
 (segment (start 125.745 97.925) (end 125.745 97.383) (width 0.2) (layer "F.Cu") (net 1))
 (segment (start 136.5 90) (end 136.5 88.75) (width 0.2) (layer "F.Cu") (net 1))
 (segment (start 121.659 93.509) (end 121.76 93.61) (width 0.2) (layer "F.Cu") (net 1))
 (segment (start 188.45 97.945) (end 188.45 96.843) (width 0.2) (layer "F.Cu") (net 1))
 (segment (start 139.26 85.99) (end 140.21 85.99) (width 0.2) (layer "F.Cu") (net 1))
 (segment (start 182.5 135.5) (end 180.275 137.725) (width 0.2) (layer "F.Cu") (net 1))
 (segment (start 196.15 97.945) (end 196.15 125.65) (width 0.2) (layer "F.Cu") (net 1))
 (segment (start 121.76 93.61) (end 122.71 93.61) (width 0.2) (layer "F.Cu") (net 1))
 (segment (start 137.9 143.2) (end 137.45 142.75) (width 0.2) (layer "F.Cu") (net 1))
 (segment (start 176.049 96.644) (end 188.349 96.644) (width 0.2) (layer "F.Cu") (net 1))
 (segment (start 163.225 138.8) (end 163.225 140.5) (width 0.2) (layer "F.Cu") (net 1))
 (segment (start 188.349 96.644) (end 188.45 96.745) (width 0.2) (layer "F.Cu") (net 1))
 (segment (start 188.45 96.745) (end 188.45 97.945) (width 0.2) (layer "F.Cu") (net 1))
 (segment (start 137.35 141.4) (end 137.45 141.5) (width 0.2) (layer "F.Cu") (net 1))
 (segment (start 168.875 138.8) (end 163.225 138.8) (width 0.2) (layer "F.Cu") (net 1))
 (segment (start 137.6 141.5) (end 138.4 141.5) (width 0.2) (layer "F.Cu") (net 1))
 (segment (start 188.649 96.644) (end 196.049 96.644) (width 0.2) (layer "F.Cu") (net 1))
 (segment (start 196.15 125.65) (end 189.85 125.65) (width 0.2) (layer "F.Cu") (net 1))
 (segment (start 121.76 85.99) (end 121.659 86.091) (width 0.2) (layer "F.Cu") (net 1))
 (segment (start 125.745 97.925) (end 125.745 103.75) (width 0.2) (layer "F.Cu") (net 1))
 (segment (start 175.85 97.945) (end 175.85 96.843) (width 0.2) (layer "F.Cu") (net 1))
 (segment (start 196.049 96.644) (end 196.15 96.745) (width 0.2) (layer "F.Cu") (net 1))
 (segment (start 121.659 86.091) (end 121.659 93.509) (width 0.2) (layer "F.Cu") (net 1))
 (segment (start 125.745 97.383) (end 123.242 94.88) (width 0.2) (layer "F.Cu") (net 1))
 (segment (start 136.5 88.75) (end 139.26 85.99) (width 0.2) (layer "F.Cu") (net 1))
 (segment (start 138.5 143.2) (end 137.9 143.2) (width 0.2) (layer "F.Cu") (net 1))
 (segment (start 131.36 92.31) (end 134.31 92.31) (width 0.2) (layer "F.Cu") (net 1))
 (segment (start 163.225 140.5) (end 139.4 140.5) (width 0.2) (layer "F.Cu") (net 1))
 (segment (start 140.21 85.99) (end 163.895 85.99) (width 0.2) (layer "F.Cu") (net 1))
 (segment (start 180.275 137.725) (end 174.8 137.725) (width 0.2) (layer "F.Cu") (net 1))
 (segment (start 163.895 85.99) (end 175.85 97.945) (width 0.2) (layer "F.Cu") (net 1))
 (segment (start 139.4 140.5) (end 138.5 141.4) (width 0.2) (layer "F.Cu") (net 1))
 (segment (start 188.45 96.843) (end 188.649 96.644) (width 0.2) (layer "F.Cu") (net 1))
 (segment (start 189.85 125.65) (end 186 129.5) (width 0.2) (layer "F.Cu") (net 1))
 (segment (start 169.95 137.725) (end 168.875 138.8) (width 0.2) (layer "F.Cu") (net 1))
 (segment (start 122.71 93.61) (end 122.71 94.88) (width 0.2) (layer "F.Cu") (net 1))
 (via (at 186 129.5) (size 0.6) (drill 0.3) (layers "F.Cu" "B.Cu") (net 1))
 (via (at 136.5 90) (size 0.6) (drill 0.3) (layers "F.Cu" "B.Cu") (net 1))
 (via (at 134.31 92.31) (size 0.6) (drill 0.3) (layers "F.Cu" "B.Cu") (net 1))
 (via (at 182.5 135.5) (size 0.6) (drill 0.3) (layers "F.Cu" "B.Cu") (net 1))
 (segment (start 134.31 92.19) (end 136.5 90) (width 0.2) (layer "B.Cu") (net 1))
 (segment (start 186 129.5) (end 182.5 133) (width 0.2) (layer "B.Cu") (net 1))
 (segment (start 134.31 92.31) (end 134.31 92.19) (width 0.2) (layer "B.Cu") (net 1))
 (segment (start 182.5 133) (end 182.5 135.5) (width 0.2) (layer "B.Cu") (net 1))
 (segment (start 122.71 91.07) (end 139.159 91.07) (width 0.2) (layer "F.Cu") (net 5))
 (segment (start 190.749 103.251) (end 194.75 99.25) (width 0.2) (layer "F.Cu") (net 5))
 (segment (start 139.159 103.251) (end 190.749 103.251) (width 0.2) (layer "F.Cu") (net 5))
 (segment (start 194.75 99.25) (end 194.75 97.945) (width 0.2) (layer "F.Cu") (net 5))
 (segment (start 139.159 91.07) (end 139.159 103.251) (width 0.2) (layer "F.Cu") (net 5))
 (segment (start 124.994 101.712) (end 124.994 125.994) (width 0.2) (layer "F.Cu") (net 10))
 (segment (start 134.5 147.5) (end 141 147.5) (width 0.2) (layer "F.Cu") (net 10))
 (segment (start 133 143) (end 133 146) (width 0.2) (layer "F.Cu") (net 10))
 (segment (start 123.242 99.96) (end 124.994 101.712) (width 0.2) (layer "F.Cu") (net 10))
 (segment (start 143 145.5) (end 143 143) (width 0.2) (layer "F.Cu") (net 10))
 (segment (start 133 146) (end 134.5 147.5) (width 0.2) (layer "F.Cu") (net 10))
 (segment (start 141 147.5) (end 143 145.5) (width 0.2) (layer "F.Cu") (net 10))
 (segment (start 122.71 99.96) (end 123.242 99.96) (width 0.2) (layer "F.Cu") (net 10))
 (segment (start 143 143) (end 142 142) (width 0.2) (layer "F.Cu") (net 10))
 (segment (start 142 142) (end 138.5 142) (width 0.2) (layer "F.Cu") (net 10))
 (segment (start 124.994 125.994) (end 133 134) (width 0.2) (layer "F.Cu") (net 10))
 (via (at 133 134) (size 0.6) (drill 0.3) (layers "F.Cu" "B.Cu") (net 10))
 (via (at 133 143) (size 0.6) (drill 0.3) (layers "F.Cu" "B.Cu") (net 10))
 (segment (start 133 134) (end 133 143) (width 0.2) (layer "B.Cu") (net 10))
 (segment (start 141 144) (end 140.5 144) (width 0.2) (layer "F.Cu") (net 4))
 (segment (start 128.5 98) (end 133.3409 98) (width 0.2) (layer "F.Cu") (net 4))
 (segment (start 140.3 143.8) (end 138.5 143.8) (width 0.2) (layer "F.Cu") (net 4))
 (segment (start 123.01 89.5) (end 126 89.5) (width 0.2) (layer "F.Cu") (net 4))
 (segment (start 141 105.6591) (end 141 134.5) (width 0.2) (layer "F.Cu") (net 4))
 (segment (start 122.71 89.8) (end 123.01 89.5) (width 0.2) (layer "F.Cu") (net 4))
 (segment (start 133.3409 98) (end 141 105.6591) (width 0.2) (layer "F.Cu") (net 4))
 (segment (start 140.5 144) (end 140.3 143.8) (width 0.2) (layer "F.Cu") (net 4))
 (via (at 126 89.5) (size 0.6) (drill 0.3) (layers "F.Cu" "B.Cu") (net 4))
 (via (at 128.5 98) (size 0.6) (drill 0.3) (layers "F.Cu" "B.Cu") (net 4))
 (via (at 141 134.5) (size 0.6) (drill 0.3) (layers "F.Cu" "B.Cu") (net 4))
 (via (at 141 144) (size 0.6) (drill 0.3) (layers "F.Cu" "B.Cu") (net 4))
 (segment (start 127 92) (end 127 96.5) (width 0.2) (layer "B.Cu") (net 4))
 (segment (start 126.5 89.5) (end 127 90) (width 0.2) (layer "B.Cu") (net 4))
 (segment (start 126 89.5) (end 126.5 89.5) (width 0.2) (layer "B.Cu") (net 4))
 (segment (start 127 96.5) (end 128.5 98) (width 0.2) (layer "B.Cu") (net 4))
 (segment (start 141 134.5) (end 141 144) (width 0.2) (layer "B.Cu") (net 4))
 (segment (start 127 90) (end 127 92) (width 0.2) (layer "B.Cu") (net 4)))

